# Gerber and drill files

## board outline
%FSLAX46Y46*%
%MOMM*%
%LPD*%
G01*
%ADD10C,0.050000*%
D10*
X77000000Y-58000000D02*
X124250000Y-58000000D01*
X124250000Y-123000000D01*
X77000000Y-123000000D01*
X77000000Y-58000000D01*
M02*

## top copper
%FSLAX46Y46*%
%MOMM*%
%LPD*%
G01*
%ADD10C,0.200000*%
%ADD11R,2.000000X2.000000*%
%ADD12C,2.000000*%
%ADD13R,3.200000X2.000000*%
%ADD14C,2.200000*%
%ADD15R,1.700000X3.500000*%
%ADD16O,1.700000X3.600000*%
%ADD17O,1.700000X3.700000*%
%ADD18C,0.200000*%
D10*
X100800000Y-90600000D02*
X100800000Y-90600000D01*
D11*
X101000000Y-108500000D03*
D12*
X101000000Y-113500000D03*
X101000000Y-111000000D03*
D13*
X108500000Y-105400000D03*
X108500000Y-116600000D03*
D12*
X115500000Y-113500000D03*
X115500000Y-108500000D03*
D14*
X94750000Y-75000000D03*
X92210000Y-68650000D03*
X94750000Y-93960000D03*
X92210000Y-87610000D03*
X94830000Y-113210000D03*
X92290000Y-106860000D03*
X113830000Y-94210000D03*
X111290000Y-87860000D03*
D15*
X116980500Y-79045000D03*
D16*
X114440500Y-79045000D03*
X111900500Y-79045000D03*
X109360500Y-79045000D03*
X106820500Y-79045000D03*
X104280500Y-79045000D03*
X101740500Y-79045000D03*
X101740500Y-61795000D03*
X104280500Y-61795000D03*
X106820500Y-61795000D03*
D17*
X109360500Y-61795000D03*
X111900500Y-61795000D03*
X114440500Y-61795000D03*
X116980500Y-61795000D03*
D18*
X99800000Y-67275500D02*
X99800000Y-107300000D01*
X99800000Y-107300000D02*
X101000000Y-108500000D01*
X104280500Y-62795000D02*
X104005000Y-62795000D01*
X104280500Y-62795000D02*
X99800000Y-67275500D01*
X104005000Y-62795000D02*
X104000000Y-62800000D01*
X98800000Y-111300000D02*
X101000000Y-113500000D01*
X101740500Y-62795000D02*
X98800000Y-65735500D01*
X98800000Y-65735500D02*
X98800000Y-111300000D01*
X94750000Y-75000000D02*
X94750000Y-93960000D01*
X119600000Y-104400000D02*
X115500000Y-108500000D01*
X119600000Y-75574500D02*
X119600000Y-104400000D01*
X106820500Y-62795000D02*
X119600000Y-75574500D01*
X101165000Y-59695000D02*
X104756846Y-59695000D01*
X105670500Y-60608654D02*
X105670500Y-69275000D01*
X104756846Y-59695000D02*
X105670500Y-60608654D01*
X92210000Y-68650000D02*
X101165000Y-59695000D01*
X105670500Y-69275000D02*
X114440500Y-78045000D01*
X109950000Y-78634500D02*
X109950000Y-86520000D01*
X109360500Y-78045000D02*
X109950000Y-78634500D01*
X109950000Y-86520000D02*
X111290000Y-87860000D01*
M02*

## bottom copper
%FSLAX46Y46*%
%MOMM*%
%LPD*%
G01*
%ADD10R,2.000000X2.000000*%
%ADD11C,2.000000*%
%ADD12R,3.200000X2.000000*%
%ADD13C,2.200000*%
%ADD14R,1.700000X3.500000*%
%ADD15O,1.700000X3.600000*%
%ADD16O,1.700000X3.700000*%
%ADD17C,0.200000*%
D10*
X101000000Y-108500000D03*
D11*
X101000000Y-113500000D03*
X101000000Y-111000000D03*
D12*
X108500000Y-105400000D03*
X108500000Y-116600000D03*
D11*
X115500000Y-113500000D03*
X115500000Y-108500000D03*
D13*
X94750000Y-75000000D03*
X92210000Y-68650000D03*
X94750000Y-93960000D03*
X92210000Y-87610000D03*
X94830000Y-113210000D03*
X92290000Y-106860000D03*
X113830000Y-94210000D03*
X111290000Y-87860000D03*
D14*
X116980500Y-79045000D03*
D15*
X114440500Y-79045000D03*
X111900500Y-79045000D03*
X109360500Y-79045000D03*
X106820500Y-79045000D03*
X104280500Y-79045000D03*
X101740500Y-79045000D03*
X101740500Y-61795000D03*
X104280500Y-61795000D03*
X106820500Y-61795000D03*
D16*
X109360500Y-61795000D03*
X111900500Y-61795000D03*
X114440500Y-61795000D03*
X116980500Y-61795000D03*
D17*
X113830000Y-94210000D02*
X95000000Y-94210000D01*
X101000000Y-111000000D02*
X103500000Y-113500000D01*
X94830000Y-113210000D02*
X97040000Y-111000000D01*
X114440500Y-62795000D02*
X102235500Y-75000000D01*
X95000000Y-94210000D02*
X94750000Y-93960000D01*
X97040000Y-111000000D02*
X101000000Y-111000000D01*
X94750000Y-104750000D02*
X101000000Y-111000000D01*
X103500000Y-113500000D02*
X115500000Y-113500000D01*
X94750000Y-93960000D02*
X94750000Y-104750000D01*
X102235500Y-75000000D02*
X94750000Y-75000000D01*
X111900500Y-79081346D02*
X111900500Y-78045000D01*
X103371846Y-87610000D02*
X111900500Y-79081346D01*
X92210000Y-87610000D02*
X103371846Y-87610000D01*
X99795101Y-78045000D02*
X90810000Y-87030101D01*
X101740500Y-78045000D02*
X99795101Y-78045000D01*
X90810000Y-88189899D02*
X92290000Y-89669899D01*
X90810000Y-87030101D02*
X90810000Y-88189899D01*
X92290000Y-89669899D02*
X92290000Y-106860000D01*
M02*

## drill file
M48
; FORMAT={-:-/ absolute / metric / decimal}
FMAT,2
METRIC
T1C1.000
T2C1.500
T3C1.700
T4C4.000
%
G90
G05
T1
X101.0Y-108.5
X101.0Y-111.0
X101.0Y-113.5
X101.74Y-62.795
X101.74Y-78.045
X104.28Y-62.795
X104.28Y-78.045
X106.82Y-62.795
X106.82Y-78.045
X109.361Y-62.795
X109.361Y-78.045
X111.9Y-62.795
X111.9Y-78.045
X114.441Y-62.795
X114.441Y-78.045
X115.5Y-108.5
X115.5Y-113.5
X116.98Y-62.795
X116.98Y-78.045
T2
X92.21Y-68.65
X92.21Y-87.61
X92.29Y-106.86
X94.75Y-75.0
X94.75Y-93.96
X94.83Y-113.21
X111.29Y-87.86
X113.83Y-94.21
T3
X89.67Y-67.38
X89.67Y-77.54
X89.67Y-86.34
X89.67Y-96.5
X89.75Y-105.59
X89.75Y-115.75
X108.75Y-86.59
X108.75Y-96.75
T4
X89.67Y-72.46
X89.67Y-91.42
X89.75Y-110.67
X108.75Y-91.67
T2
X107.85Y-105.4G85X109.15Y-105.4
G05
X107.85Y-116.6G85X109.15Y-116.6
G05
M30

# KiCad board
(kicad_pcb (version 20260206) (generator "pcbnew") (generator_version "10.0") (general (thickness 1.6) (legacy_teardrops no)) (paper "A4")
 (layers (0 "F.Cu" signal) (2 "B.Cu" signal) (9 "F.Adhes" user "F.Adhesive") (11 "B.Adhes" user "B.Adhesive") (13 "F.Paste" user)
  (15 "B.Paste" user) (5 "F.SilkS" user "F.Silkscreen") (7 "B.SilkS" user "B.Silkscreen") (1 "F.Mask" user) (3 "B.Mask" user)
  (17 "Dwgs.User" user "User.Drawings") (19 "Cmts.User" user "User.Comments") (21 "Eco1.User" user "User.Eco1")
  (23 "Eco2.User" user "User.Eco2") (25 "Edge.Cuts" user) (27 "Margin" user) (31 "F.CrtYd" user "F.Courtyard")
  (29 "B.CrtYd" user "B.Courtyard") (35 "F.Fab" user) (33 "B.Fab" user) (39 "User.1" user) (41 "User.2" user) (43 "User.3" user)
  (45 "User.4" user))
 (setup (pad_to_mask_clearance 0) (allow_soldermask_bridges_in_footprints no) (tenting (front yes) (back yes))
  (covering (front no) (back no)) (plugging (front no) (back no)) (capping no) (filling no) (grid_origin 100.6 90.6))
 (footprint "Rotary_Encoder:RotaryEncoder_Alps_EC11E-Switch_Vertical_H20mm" (layer "F.Cu") (at 101 108.5)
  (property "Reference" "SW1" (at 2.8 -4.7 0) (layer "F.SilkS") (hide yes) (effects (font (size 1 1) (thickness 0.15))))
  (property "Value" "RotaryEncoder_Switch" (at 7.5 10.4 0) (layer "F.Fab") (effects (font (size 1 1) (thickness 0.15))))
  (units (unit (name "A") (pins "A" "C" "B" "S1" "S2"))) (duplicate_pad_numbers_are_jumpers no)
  (pad "A" thru_hole rect (at 0 0) (size 2 2) (drill 1) (layers "*.Cu" "*.Mask") (remove_unused_layers no) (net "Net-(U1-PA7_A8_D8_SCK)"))
  (pad "B" thru_hole circle (at 0 5) (size 2 2) (drill 1) (layers "*.Cu" "*.Mask") (remove_unused_layers no) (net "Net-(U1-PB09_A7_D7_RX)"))
  (pad "C" thru_hole circle (at 0 2.5) (size 2 2) (drill 1) (layers "*.Cu" "*.Mask") (remove_unused_layers no) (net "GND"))
  (pad "MP" thru_hole rect (at 7.5 -3.1) (size 3.2 2) (drill oval 2.8 1.5) (layers "*.Cu" "*.Mask") (remove_unused_layers no))
  (pad "MP" thru_hole rect (at 7.5 8.1) (size 3.2 2) (drill oval 2.8 1.5) (layers "*.Cu" "*.Mask") (remove_unused_layers no))
  (pad "S1" thru_hole circle (at 14.5 5) (size 2 2) (drill 1) (layers "*.Cu" "*.Mask") (remove_unused_layers no) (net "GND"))
  (pad "S2" thru_hole circle (at 14.5 0) (size 2 2) (drill 1) (layers "*.Cu" "*.Mask") (remove_unused_layers no)
   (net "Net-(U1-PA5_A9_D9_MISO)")))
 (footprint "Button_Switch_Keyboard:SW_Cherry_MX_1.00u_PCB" (layer "F.Cu") (at 94.75 75 -90)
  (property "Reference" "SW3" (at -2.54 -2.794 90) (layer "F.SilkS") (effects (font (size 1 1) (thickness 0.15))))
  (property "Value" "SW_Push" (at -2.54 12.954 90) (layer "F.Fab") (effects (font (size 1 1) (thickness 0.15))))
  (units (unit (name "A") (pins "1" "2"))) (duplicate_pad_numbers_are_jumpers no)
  (pad "" np_thru_hole circle (at -7.62 5.08 270) (size 1.7 1.7) (drill 1.7) (layers "*.Cu" "*.Mask"))
  (pad "" np_thru_hole circle (at -2.54 5.08 270) (size 4 4) (drill 4) (layers "*.Cu" "*.Mask"))
  (pad "" np_thru_hole circle (at 2.54 5.08 270) (size 1.7 1.7) (drill 1.7) (layers "*.Cu" "*.Mask"))
  (pad "1" thru_hole circle (at 0 0 270) (size 2.2 2.2) (drill 1.5) (layers "*.Cu" "*.Mask") (remove_unused_layers no) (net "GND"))
  (pad "2" thru_hole circle (at -6.35 2.54 270) (size 2.2 2.2) (drill 1.5) (layers "*.Cu" "*.Mask") (remove_unused_layers no)
   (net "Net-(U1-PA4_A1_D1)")))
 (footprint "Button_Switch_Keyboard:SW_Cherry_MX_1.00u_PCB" (layer "F.Cu") (at 94.75 93.96 -90)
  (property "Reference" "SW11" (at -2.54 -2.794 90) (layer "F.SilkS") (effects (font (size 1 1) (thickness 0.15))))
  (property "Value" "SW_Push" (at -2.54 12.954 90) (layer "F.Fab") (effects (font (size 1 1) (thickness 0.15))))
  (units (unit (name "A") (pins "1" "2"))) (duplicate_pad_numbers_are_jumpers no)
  (pad "" np_thru_hole circle (at -7.62 5.08 270) (size 1.7 1.7) (drill 1.7) (layers "*.Cu" "*.Mask"))
  (pad "" np_thru_hole circle (at -2.54 5.08 270) (size 4 4) (drill 4) (layers "*.Cu" "*.Mask"))
  (pad "" np_thru_hole circle (at 2.54 5.08 270) (size 1.7 1.7) (drill 1.7) (layers "*.Cu" "*.Mask"))
  (pad "1" thru_hole circle (at 0 0 270) (size 2.2 2.2) (drill 1.5) (layers "*.Cu" "*.Mask") (remove_unused_layers no) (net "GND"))
  (pad "2" thru_hole circle (at -6.35 2.54 270) (size 2.2 2.2) (drill 1.5) (layers "*.Cu" "*.Mask") (remove_unused_layers no)
   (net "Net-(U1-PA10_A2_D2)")))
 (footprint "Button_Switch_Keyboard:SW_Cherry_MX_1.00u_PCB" (layer "F.Cu") (at 94.83 113.21 -90)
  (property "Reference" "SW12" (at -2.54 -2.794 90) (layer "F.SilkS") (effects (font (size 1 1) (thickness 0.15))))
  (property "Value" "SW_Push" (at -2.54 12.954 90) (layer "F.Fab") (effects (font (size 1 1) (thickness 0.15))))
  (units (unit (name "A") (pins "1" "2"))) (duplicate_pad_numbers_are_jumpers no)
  (pad "" np_thru_hole circle (at -7.62 5.08 270) (size 1.7 1.7) (drill 1.7) (layers "*.Cu" "*.Mask"))
  (pad "" np_thru_hole circle (at -2.54 5.08 270) (size 4 4) (drill 4) (layers "*.Cu" "*.Mask"))
  (pad "" np_thru_hole circle (at 2.54 5.08 270) (size 1.7 1.7) (drill 1.7) (layers "*.Cu" "*.Mask"))
  (pad "1" thru_hole circle (at 0 0 270) (size 2.2 2.2) (drill 1.5) (layers "*.Cu" "*.Mask") (remove_unused_layers no) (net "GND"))
  (pad "2" thru_hole circle (at -6.35 2.54 270) (size 2.2 2.2) (drill 1.5) (layers "*.Cu" "*.Mask") (remove_unused_layers no)
   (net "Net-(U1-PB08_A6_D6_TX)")))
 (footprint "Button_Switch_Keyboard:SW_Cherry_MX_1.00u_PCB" (layer "F.Cu") (at 113.83 94.21 -90)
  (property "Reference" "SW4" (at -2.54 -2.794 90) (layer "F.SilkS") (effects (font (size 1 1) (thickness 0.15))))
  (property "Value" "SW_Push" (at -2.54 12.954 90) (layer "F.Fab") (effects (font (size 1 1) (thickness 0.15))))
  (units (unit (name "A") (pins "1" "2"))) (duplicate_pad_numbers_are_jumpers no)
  (pad "" np_thru_hole circle (at -7.62 5.08 270) (size 1.7 1.7) (drill 1.7) (layers "*.Cu" "*.Mask"))
  (pad "" np_thru_hole circle (at -2.54 5.08 270) (size 4 4) (drill 4) (layers "*.Cu" "*.Mask"))
  (pad "" np_thru_hole circle (at 2.54 5.08 270) (size 1.7 1.7) (drill 1.7) (layers "*.Cu" "*.Mask"))
  (pad "1" thru_hole circle (at 0 0 270) (size 2.2 2.2) (drill 1.5) (layers "*.Cu" "*.Mask") (remove_unused_layers no) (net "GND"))
  (pad "2" thru_hole circle (at -6.35 2.54 270) (size 2.2 2.2) (drill 1.5) (layers "*.Cu" "*.Mask") (remove_unused_layers no)
   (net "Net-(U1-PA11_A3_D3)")))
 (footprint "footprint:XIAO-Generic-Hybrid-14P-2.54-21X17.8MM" (layer "B.Cu") (at 109.3605 70.42 90)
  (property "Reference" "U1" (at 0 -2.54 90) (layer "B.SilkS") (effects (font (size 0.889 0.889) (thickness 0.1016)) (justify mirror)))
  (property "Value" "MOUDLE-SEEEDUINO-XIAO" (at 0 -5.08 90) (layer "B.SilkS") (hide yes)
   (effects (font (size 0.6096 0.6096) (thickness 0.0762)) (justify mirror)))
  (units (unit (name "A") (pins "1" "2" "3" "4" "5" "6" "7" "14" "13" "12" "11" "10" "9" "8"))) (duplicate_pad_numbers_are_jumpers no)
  (pad "1" thru_hole rect (at -7.625 7.62 90) (size 3.5 1.7) (drill 1 (offset -1 0)) (layers "*.Cu" "*.Mask") (remove_unused_layers no)
   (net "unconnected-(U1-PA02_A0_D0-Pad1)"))
  (pad "2" thru_hole oval (at -7.625 5.08 90) (size 3.6 1.7) (drill 1 (offset -1 0)) (layers "*.Cu" "*.Mask") (remove_unused_layers no)
   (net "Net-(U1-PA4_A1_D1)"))
  (pad "3" thru_hole oval (at -7.625 2.54 90) (size 3.6 1.7) (drill 1 (offset -1 0)) (layers "*.Cu" "*.Mask") (remove_unused_layers no)
   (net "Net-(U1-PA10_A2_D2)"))
  (pad "4" thru_hole oval (at -7.625 0 90) (size 3.6 1.7) (drill 1 (offset -1 0)) (layers "*.Cu" "*.Mask") (remove_unused_layers no)
   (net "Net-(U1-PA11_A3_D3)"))
  (pad "5" thru_hole oval (at -7.625 -2.54 90) (size 3.6 1.7) (drill 1 (offset -1 0)) (layers "*.Cu" "*.Mask") (remove_unused_layers no)
   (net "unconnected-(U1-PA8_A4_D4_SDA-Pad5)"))
  (pad "6" thru_hole oval (at -7.625 -5.08 270) (size 3.6 1.7) (drill 1 (offset 1 0)) (layers "*.Cu" "*.Mask") (remove_unused_layers no)
   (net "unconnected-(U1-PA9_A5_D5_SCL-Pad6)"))
  (pad "7" thru_hole oval (at -7.625 -7.62 90) (size 3.6 1.7) (drill 1 (offset -1 0)) (layers "*.Cu" "*.Mask") (remove_unused_layers no)
   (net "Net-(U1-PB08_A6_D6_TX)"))
  (pad "8" thru_hole oval (at 7.625 -7.62 90) (size 3.6 1.7) (drill 1 (offset 1 0)) (layers "*.Cu" "*.Mask") (remove_unused_layers no)
   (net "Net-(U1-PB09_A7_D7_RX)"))
  (pad "9" thru_hole oval (at 7.625 -5.08 90) (size 3.6 1.7) (drill 1 (offset 1 0)) (layers "*.Cu" "*.Mask") (remove_unused_layers no)
   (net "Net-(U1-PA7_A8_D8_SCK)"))
  (pad "10" thru_hole oval (at 7.625 -2.54 90) (size 3.6 1.7) (drill 1 (offset 1 0)) (layers "*.Cu" "*.Mask") (remove_unused_layers no)
   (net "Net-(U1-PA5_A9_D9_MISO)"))
  (pad "11" thru_hole oval (at 7.625 0 90) (size 3.7 1.7) (drill 1 (offset 1 0)) (layers "*.Cu" "*.Mask") (remove_unused_layers no)
   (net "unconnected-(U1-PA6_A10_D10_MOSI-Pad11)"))
  (pad "12" thru_hole oval (at 7.625 2.54 90) (size 3.7 1.7) (drill 1 (offset 1 0)) (layers "*.Cu" "*.Mask") (remove_unused_layers no)
   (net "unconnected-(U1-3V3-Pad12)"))
  (pad "13" thru_hole oval (at 7.625 5.08 90) (size 3.7 1.7) (drill 1 (offset 1 0)) (layers "*.Cu" "*.Mask") (remove_unused_layers no)
   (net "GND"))
  (pad "14" thru_hole oval (at 7.625 7.62 90) (size 3.7 1.7) (drill 1 (offset 1 0)) (layers "*.Cu" "*.Mask") (remove_unused_layers no)
   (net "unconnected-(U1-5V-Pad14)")))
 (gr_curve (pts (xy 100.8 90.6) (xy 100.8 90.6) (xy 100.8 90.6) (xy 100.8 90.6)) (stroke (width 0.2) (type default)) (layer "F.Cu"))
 (gr_rect (start 77 58) (end 124.25 123) (stroke (width 0.05) (type default)) (fill no) (layer "Edge.Cuts"))
 (segment (start 99.8 67.2755) (end 99.8 107.3) (width 0.2) (layer "F.Cu") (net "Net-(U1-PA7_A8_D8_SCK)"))
 (segment (start 99.8 107.3) (end 101 108.5) (width 0.2) (layer "F.Cu") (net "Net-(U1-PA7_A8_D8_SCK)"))
 (segment (start 104.2805 62.795) (end 104.005 62.795) (width 0.2) (layer "F.Cu") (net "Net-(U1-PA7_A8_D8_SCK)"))
 (segment (start 104.2805 62.795) (end 99.8 67.2755) (width 0.2) (layer "F.Cu") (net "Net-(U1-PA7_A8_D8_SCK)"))
 (segment (start 104.005 62.795) (end 104 62.8) (width 0.2) (layer "F.Cu") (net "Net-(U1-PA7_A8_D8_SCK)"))
 (segment (start 98.8 111.3) (end 101 113.5) (width 0.2) (layer "F.Cu") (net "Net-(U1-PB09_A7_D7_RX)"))
 (segment (start 101.7405 62.795) (end 98.8 65.7355) (width 0.2) (layer "F.Cu") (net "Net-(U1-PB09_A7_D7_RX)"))
 (segment (start 98.8 65.7355) (end 98.8 111.3) (width 0.2) (layer "F.Cu") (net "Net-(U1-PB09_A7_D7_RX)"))
 (segment (start 94.75 75) (end 94.75 93.96) (width 0.2) (layer "F.Cu") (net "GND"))
 (segment (start 113.83 94.21) (end 95 94.21) (width 0.2) (layer "B.Cu") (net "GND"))
 (segment (start 101 111) (end 103.5 113.5) (width 0.2) (layer "B.Cu") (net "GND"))
 (segment (start 94.83 113.21) (end 97.04 111) (width 0.2) (layer "B.Cu") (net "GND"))
 (segment (start 114.4405 62.795) (end 102.2355 75) (width 0.2) (layer "B.Cu") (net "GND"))
 (segment (start 95 94.21) (end 94.75 93.96) (width 0.2) (layer "B.Cu") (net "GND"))
 (segment (start 97.04 111) (end 101 111) (width 0.2) (layer "B.Cu") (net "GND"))
 (segment (start 94.75 104.75) (end 101 111) (width 0.2) (layer "B.Cu") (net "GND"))
 (segment (start 103.5 113.5) (end 115.5 113.5) (width 0.2) (layer "B.Cu") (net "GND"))
 (segment (start 94.75 93.96) (end 94.75 104.75) (width 0.2) (layer "B.Cu") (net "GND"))
 (segment (start 102.2355 75) (end 94.75 75) (width 0.2) (layer "B.Cu") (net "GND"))
 (segment (start 119.6 104.4) (end 115.5 108.5) (width 0.2) (layer "F.Cu") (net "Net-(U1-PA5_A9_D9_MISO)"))
 (segment (start 119.6 75.5745) (end 119.6 104.4) (width 0.2) (layer "F.Cu") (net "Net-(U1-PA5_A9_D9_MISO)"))
 (segment (start 106.8205 62.795) (end 119.6 75.5745) (width 0.2) (layer "F.Cu") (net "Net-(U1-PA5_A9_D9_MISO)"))
 (segment (start 101.165 59.695) (end 104.756846 59.695) (width 0.2) (layer "F.Cu") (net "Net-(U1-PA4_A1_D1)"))
 (segment (start 105.6705 60.608654) (end 105.6705 69.275) (width 0.2) (layer "F.Cu") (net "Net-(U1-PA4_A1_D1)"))
 (segment (start 104.756846 59.695) (end 105.6705 60.608654) (width 0.2) (layer "F.Cu") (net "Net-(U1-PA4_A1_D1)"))
 (segment (start 92.21 68.65) (end 101.165 59.695) (width 0.2) (layer "F.Cu") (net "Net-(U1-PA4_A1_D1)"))
 (segment (start 105.6705 69.275) (end 114.4405 78.045) (width 0.2) (layer "F.Cu") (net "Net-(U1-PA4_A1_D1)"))
 (segment (start 111.9005 79.081346) (end 111.9005 78.045) (width 0.2) (layer "B.Cu") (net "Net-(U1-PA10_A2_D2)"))
 (segment (start 103.371846 87.61) (end 111.9005 79.081346) (width 0.2) (layer "B.Cu") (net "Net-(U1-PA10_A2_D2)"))
 (segment (start 92.21 87.61) (end 103.371846 87.61) (width 0.2) (layer "B.Cu") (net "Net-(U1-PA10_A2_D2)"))
 (segment (start 99.795101 78.045) (end 90.81 87.030101) (width 0.2) (layer "B.Cu") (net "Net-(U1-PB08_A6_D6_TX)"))
 (segment (start 101.7405 78.045) (end 99.795101 78.045) (width 0.2) (layer "B.Cu") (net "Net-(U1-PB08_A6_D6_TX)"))
 (segment (start 90.81 88.189899) (end 92.29 89.669899) (width 0.2) (layer "B.Cu") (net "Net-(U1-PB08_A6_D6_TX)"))
 (segment (start 90.81 87.030101) (end 90.81 88.189899) (width 0.2) (layer "B.Cu") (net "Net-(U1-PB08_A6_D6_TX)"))
 (segment (start 92.29 89.669899) (end 92.29 106.86) (width 0.2) (layer "B.Cu") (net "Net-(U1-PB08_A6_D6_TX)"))
 (segment (start 109.95 78.6345) (end 109.95 86.52) (width 0.2) (layer "F.Cu") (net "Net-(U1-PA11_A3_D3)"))
 (segment (start 109.3605 78.045) (end 109.95 78.6345) (width 0.2) (layer "F.Cu") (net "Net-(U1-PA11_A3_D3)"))
 (segment (start 109.95 86.52) (end 111.29 87.86) (width 0.2) (layer "F.Cu") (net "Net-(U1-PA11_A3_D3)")))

